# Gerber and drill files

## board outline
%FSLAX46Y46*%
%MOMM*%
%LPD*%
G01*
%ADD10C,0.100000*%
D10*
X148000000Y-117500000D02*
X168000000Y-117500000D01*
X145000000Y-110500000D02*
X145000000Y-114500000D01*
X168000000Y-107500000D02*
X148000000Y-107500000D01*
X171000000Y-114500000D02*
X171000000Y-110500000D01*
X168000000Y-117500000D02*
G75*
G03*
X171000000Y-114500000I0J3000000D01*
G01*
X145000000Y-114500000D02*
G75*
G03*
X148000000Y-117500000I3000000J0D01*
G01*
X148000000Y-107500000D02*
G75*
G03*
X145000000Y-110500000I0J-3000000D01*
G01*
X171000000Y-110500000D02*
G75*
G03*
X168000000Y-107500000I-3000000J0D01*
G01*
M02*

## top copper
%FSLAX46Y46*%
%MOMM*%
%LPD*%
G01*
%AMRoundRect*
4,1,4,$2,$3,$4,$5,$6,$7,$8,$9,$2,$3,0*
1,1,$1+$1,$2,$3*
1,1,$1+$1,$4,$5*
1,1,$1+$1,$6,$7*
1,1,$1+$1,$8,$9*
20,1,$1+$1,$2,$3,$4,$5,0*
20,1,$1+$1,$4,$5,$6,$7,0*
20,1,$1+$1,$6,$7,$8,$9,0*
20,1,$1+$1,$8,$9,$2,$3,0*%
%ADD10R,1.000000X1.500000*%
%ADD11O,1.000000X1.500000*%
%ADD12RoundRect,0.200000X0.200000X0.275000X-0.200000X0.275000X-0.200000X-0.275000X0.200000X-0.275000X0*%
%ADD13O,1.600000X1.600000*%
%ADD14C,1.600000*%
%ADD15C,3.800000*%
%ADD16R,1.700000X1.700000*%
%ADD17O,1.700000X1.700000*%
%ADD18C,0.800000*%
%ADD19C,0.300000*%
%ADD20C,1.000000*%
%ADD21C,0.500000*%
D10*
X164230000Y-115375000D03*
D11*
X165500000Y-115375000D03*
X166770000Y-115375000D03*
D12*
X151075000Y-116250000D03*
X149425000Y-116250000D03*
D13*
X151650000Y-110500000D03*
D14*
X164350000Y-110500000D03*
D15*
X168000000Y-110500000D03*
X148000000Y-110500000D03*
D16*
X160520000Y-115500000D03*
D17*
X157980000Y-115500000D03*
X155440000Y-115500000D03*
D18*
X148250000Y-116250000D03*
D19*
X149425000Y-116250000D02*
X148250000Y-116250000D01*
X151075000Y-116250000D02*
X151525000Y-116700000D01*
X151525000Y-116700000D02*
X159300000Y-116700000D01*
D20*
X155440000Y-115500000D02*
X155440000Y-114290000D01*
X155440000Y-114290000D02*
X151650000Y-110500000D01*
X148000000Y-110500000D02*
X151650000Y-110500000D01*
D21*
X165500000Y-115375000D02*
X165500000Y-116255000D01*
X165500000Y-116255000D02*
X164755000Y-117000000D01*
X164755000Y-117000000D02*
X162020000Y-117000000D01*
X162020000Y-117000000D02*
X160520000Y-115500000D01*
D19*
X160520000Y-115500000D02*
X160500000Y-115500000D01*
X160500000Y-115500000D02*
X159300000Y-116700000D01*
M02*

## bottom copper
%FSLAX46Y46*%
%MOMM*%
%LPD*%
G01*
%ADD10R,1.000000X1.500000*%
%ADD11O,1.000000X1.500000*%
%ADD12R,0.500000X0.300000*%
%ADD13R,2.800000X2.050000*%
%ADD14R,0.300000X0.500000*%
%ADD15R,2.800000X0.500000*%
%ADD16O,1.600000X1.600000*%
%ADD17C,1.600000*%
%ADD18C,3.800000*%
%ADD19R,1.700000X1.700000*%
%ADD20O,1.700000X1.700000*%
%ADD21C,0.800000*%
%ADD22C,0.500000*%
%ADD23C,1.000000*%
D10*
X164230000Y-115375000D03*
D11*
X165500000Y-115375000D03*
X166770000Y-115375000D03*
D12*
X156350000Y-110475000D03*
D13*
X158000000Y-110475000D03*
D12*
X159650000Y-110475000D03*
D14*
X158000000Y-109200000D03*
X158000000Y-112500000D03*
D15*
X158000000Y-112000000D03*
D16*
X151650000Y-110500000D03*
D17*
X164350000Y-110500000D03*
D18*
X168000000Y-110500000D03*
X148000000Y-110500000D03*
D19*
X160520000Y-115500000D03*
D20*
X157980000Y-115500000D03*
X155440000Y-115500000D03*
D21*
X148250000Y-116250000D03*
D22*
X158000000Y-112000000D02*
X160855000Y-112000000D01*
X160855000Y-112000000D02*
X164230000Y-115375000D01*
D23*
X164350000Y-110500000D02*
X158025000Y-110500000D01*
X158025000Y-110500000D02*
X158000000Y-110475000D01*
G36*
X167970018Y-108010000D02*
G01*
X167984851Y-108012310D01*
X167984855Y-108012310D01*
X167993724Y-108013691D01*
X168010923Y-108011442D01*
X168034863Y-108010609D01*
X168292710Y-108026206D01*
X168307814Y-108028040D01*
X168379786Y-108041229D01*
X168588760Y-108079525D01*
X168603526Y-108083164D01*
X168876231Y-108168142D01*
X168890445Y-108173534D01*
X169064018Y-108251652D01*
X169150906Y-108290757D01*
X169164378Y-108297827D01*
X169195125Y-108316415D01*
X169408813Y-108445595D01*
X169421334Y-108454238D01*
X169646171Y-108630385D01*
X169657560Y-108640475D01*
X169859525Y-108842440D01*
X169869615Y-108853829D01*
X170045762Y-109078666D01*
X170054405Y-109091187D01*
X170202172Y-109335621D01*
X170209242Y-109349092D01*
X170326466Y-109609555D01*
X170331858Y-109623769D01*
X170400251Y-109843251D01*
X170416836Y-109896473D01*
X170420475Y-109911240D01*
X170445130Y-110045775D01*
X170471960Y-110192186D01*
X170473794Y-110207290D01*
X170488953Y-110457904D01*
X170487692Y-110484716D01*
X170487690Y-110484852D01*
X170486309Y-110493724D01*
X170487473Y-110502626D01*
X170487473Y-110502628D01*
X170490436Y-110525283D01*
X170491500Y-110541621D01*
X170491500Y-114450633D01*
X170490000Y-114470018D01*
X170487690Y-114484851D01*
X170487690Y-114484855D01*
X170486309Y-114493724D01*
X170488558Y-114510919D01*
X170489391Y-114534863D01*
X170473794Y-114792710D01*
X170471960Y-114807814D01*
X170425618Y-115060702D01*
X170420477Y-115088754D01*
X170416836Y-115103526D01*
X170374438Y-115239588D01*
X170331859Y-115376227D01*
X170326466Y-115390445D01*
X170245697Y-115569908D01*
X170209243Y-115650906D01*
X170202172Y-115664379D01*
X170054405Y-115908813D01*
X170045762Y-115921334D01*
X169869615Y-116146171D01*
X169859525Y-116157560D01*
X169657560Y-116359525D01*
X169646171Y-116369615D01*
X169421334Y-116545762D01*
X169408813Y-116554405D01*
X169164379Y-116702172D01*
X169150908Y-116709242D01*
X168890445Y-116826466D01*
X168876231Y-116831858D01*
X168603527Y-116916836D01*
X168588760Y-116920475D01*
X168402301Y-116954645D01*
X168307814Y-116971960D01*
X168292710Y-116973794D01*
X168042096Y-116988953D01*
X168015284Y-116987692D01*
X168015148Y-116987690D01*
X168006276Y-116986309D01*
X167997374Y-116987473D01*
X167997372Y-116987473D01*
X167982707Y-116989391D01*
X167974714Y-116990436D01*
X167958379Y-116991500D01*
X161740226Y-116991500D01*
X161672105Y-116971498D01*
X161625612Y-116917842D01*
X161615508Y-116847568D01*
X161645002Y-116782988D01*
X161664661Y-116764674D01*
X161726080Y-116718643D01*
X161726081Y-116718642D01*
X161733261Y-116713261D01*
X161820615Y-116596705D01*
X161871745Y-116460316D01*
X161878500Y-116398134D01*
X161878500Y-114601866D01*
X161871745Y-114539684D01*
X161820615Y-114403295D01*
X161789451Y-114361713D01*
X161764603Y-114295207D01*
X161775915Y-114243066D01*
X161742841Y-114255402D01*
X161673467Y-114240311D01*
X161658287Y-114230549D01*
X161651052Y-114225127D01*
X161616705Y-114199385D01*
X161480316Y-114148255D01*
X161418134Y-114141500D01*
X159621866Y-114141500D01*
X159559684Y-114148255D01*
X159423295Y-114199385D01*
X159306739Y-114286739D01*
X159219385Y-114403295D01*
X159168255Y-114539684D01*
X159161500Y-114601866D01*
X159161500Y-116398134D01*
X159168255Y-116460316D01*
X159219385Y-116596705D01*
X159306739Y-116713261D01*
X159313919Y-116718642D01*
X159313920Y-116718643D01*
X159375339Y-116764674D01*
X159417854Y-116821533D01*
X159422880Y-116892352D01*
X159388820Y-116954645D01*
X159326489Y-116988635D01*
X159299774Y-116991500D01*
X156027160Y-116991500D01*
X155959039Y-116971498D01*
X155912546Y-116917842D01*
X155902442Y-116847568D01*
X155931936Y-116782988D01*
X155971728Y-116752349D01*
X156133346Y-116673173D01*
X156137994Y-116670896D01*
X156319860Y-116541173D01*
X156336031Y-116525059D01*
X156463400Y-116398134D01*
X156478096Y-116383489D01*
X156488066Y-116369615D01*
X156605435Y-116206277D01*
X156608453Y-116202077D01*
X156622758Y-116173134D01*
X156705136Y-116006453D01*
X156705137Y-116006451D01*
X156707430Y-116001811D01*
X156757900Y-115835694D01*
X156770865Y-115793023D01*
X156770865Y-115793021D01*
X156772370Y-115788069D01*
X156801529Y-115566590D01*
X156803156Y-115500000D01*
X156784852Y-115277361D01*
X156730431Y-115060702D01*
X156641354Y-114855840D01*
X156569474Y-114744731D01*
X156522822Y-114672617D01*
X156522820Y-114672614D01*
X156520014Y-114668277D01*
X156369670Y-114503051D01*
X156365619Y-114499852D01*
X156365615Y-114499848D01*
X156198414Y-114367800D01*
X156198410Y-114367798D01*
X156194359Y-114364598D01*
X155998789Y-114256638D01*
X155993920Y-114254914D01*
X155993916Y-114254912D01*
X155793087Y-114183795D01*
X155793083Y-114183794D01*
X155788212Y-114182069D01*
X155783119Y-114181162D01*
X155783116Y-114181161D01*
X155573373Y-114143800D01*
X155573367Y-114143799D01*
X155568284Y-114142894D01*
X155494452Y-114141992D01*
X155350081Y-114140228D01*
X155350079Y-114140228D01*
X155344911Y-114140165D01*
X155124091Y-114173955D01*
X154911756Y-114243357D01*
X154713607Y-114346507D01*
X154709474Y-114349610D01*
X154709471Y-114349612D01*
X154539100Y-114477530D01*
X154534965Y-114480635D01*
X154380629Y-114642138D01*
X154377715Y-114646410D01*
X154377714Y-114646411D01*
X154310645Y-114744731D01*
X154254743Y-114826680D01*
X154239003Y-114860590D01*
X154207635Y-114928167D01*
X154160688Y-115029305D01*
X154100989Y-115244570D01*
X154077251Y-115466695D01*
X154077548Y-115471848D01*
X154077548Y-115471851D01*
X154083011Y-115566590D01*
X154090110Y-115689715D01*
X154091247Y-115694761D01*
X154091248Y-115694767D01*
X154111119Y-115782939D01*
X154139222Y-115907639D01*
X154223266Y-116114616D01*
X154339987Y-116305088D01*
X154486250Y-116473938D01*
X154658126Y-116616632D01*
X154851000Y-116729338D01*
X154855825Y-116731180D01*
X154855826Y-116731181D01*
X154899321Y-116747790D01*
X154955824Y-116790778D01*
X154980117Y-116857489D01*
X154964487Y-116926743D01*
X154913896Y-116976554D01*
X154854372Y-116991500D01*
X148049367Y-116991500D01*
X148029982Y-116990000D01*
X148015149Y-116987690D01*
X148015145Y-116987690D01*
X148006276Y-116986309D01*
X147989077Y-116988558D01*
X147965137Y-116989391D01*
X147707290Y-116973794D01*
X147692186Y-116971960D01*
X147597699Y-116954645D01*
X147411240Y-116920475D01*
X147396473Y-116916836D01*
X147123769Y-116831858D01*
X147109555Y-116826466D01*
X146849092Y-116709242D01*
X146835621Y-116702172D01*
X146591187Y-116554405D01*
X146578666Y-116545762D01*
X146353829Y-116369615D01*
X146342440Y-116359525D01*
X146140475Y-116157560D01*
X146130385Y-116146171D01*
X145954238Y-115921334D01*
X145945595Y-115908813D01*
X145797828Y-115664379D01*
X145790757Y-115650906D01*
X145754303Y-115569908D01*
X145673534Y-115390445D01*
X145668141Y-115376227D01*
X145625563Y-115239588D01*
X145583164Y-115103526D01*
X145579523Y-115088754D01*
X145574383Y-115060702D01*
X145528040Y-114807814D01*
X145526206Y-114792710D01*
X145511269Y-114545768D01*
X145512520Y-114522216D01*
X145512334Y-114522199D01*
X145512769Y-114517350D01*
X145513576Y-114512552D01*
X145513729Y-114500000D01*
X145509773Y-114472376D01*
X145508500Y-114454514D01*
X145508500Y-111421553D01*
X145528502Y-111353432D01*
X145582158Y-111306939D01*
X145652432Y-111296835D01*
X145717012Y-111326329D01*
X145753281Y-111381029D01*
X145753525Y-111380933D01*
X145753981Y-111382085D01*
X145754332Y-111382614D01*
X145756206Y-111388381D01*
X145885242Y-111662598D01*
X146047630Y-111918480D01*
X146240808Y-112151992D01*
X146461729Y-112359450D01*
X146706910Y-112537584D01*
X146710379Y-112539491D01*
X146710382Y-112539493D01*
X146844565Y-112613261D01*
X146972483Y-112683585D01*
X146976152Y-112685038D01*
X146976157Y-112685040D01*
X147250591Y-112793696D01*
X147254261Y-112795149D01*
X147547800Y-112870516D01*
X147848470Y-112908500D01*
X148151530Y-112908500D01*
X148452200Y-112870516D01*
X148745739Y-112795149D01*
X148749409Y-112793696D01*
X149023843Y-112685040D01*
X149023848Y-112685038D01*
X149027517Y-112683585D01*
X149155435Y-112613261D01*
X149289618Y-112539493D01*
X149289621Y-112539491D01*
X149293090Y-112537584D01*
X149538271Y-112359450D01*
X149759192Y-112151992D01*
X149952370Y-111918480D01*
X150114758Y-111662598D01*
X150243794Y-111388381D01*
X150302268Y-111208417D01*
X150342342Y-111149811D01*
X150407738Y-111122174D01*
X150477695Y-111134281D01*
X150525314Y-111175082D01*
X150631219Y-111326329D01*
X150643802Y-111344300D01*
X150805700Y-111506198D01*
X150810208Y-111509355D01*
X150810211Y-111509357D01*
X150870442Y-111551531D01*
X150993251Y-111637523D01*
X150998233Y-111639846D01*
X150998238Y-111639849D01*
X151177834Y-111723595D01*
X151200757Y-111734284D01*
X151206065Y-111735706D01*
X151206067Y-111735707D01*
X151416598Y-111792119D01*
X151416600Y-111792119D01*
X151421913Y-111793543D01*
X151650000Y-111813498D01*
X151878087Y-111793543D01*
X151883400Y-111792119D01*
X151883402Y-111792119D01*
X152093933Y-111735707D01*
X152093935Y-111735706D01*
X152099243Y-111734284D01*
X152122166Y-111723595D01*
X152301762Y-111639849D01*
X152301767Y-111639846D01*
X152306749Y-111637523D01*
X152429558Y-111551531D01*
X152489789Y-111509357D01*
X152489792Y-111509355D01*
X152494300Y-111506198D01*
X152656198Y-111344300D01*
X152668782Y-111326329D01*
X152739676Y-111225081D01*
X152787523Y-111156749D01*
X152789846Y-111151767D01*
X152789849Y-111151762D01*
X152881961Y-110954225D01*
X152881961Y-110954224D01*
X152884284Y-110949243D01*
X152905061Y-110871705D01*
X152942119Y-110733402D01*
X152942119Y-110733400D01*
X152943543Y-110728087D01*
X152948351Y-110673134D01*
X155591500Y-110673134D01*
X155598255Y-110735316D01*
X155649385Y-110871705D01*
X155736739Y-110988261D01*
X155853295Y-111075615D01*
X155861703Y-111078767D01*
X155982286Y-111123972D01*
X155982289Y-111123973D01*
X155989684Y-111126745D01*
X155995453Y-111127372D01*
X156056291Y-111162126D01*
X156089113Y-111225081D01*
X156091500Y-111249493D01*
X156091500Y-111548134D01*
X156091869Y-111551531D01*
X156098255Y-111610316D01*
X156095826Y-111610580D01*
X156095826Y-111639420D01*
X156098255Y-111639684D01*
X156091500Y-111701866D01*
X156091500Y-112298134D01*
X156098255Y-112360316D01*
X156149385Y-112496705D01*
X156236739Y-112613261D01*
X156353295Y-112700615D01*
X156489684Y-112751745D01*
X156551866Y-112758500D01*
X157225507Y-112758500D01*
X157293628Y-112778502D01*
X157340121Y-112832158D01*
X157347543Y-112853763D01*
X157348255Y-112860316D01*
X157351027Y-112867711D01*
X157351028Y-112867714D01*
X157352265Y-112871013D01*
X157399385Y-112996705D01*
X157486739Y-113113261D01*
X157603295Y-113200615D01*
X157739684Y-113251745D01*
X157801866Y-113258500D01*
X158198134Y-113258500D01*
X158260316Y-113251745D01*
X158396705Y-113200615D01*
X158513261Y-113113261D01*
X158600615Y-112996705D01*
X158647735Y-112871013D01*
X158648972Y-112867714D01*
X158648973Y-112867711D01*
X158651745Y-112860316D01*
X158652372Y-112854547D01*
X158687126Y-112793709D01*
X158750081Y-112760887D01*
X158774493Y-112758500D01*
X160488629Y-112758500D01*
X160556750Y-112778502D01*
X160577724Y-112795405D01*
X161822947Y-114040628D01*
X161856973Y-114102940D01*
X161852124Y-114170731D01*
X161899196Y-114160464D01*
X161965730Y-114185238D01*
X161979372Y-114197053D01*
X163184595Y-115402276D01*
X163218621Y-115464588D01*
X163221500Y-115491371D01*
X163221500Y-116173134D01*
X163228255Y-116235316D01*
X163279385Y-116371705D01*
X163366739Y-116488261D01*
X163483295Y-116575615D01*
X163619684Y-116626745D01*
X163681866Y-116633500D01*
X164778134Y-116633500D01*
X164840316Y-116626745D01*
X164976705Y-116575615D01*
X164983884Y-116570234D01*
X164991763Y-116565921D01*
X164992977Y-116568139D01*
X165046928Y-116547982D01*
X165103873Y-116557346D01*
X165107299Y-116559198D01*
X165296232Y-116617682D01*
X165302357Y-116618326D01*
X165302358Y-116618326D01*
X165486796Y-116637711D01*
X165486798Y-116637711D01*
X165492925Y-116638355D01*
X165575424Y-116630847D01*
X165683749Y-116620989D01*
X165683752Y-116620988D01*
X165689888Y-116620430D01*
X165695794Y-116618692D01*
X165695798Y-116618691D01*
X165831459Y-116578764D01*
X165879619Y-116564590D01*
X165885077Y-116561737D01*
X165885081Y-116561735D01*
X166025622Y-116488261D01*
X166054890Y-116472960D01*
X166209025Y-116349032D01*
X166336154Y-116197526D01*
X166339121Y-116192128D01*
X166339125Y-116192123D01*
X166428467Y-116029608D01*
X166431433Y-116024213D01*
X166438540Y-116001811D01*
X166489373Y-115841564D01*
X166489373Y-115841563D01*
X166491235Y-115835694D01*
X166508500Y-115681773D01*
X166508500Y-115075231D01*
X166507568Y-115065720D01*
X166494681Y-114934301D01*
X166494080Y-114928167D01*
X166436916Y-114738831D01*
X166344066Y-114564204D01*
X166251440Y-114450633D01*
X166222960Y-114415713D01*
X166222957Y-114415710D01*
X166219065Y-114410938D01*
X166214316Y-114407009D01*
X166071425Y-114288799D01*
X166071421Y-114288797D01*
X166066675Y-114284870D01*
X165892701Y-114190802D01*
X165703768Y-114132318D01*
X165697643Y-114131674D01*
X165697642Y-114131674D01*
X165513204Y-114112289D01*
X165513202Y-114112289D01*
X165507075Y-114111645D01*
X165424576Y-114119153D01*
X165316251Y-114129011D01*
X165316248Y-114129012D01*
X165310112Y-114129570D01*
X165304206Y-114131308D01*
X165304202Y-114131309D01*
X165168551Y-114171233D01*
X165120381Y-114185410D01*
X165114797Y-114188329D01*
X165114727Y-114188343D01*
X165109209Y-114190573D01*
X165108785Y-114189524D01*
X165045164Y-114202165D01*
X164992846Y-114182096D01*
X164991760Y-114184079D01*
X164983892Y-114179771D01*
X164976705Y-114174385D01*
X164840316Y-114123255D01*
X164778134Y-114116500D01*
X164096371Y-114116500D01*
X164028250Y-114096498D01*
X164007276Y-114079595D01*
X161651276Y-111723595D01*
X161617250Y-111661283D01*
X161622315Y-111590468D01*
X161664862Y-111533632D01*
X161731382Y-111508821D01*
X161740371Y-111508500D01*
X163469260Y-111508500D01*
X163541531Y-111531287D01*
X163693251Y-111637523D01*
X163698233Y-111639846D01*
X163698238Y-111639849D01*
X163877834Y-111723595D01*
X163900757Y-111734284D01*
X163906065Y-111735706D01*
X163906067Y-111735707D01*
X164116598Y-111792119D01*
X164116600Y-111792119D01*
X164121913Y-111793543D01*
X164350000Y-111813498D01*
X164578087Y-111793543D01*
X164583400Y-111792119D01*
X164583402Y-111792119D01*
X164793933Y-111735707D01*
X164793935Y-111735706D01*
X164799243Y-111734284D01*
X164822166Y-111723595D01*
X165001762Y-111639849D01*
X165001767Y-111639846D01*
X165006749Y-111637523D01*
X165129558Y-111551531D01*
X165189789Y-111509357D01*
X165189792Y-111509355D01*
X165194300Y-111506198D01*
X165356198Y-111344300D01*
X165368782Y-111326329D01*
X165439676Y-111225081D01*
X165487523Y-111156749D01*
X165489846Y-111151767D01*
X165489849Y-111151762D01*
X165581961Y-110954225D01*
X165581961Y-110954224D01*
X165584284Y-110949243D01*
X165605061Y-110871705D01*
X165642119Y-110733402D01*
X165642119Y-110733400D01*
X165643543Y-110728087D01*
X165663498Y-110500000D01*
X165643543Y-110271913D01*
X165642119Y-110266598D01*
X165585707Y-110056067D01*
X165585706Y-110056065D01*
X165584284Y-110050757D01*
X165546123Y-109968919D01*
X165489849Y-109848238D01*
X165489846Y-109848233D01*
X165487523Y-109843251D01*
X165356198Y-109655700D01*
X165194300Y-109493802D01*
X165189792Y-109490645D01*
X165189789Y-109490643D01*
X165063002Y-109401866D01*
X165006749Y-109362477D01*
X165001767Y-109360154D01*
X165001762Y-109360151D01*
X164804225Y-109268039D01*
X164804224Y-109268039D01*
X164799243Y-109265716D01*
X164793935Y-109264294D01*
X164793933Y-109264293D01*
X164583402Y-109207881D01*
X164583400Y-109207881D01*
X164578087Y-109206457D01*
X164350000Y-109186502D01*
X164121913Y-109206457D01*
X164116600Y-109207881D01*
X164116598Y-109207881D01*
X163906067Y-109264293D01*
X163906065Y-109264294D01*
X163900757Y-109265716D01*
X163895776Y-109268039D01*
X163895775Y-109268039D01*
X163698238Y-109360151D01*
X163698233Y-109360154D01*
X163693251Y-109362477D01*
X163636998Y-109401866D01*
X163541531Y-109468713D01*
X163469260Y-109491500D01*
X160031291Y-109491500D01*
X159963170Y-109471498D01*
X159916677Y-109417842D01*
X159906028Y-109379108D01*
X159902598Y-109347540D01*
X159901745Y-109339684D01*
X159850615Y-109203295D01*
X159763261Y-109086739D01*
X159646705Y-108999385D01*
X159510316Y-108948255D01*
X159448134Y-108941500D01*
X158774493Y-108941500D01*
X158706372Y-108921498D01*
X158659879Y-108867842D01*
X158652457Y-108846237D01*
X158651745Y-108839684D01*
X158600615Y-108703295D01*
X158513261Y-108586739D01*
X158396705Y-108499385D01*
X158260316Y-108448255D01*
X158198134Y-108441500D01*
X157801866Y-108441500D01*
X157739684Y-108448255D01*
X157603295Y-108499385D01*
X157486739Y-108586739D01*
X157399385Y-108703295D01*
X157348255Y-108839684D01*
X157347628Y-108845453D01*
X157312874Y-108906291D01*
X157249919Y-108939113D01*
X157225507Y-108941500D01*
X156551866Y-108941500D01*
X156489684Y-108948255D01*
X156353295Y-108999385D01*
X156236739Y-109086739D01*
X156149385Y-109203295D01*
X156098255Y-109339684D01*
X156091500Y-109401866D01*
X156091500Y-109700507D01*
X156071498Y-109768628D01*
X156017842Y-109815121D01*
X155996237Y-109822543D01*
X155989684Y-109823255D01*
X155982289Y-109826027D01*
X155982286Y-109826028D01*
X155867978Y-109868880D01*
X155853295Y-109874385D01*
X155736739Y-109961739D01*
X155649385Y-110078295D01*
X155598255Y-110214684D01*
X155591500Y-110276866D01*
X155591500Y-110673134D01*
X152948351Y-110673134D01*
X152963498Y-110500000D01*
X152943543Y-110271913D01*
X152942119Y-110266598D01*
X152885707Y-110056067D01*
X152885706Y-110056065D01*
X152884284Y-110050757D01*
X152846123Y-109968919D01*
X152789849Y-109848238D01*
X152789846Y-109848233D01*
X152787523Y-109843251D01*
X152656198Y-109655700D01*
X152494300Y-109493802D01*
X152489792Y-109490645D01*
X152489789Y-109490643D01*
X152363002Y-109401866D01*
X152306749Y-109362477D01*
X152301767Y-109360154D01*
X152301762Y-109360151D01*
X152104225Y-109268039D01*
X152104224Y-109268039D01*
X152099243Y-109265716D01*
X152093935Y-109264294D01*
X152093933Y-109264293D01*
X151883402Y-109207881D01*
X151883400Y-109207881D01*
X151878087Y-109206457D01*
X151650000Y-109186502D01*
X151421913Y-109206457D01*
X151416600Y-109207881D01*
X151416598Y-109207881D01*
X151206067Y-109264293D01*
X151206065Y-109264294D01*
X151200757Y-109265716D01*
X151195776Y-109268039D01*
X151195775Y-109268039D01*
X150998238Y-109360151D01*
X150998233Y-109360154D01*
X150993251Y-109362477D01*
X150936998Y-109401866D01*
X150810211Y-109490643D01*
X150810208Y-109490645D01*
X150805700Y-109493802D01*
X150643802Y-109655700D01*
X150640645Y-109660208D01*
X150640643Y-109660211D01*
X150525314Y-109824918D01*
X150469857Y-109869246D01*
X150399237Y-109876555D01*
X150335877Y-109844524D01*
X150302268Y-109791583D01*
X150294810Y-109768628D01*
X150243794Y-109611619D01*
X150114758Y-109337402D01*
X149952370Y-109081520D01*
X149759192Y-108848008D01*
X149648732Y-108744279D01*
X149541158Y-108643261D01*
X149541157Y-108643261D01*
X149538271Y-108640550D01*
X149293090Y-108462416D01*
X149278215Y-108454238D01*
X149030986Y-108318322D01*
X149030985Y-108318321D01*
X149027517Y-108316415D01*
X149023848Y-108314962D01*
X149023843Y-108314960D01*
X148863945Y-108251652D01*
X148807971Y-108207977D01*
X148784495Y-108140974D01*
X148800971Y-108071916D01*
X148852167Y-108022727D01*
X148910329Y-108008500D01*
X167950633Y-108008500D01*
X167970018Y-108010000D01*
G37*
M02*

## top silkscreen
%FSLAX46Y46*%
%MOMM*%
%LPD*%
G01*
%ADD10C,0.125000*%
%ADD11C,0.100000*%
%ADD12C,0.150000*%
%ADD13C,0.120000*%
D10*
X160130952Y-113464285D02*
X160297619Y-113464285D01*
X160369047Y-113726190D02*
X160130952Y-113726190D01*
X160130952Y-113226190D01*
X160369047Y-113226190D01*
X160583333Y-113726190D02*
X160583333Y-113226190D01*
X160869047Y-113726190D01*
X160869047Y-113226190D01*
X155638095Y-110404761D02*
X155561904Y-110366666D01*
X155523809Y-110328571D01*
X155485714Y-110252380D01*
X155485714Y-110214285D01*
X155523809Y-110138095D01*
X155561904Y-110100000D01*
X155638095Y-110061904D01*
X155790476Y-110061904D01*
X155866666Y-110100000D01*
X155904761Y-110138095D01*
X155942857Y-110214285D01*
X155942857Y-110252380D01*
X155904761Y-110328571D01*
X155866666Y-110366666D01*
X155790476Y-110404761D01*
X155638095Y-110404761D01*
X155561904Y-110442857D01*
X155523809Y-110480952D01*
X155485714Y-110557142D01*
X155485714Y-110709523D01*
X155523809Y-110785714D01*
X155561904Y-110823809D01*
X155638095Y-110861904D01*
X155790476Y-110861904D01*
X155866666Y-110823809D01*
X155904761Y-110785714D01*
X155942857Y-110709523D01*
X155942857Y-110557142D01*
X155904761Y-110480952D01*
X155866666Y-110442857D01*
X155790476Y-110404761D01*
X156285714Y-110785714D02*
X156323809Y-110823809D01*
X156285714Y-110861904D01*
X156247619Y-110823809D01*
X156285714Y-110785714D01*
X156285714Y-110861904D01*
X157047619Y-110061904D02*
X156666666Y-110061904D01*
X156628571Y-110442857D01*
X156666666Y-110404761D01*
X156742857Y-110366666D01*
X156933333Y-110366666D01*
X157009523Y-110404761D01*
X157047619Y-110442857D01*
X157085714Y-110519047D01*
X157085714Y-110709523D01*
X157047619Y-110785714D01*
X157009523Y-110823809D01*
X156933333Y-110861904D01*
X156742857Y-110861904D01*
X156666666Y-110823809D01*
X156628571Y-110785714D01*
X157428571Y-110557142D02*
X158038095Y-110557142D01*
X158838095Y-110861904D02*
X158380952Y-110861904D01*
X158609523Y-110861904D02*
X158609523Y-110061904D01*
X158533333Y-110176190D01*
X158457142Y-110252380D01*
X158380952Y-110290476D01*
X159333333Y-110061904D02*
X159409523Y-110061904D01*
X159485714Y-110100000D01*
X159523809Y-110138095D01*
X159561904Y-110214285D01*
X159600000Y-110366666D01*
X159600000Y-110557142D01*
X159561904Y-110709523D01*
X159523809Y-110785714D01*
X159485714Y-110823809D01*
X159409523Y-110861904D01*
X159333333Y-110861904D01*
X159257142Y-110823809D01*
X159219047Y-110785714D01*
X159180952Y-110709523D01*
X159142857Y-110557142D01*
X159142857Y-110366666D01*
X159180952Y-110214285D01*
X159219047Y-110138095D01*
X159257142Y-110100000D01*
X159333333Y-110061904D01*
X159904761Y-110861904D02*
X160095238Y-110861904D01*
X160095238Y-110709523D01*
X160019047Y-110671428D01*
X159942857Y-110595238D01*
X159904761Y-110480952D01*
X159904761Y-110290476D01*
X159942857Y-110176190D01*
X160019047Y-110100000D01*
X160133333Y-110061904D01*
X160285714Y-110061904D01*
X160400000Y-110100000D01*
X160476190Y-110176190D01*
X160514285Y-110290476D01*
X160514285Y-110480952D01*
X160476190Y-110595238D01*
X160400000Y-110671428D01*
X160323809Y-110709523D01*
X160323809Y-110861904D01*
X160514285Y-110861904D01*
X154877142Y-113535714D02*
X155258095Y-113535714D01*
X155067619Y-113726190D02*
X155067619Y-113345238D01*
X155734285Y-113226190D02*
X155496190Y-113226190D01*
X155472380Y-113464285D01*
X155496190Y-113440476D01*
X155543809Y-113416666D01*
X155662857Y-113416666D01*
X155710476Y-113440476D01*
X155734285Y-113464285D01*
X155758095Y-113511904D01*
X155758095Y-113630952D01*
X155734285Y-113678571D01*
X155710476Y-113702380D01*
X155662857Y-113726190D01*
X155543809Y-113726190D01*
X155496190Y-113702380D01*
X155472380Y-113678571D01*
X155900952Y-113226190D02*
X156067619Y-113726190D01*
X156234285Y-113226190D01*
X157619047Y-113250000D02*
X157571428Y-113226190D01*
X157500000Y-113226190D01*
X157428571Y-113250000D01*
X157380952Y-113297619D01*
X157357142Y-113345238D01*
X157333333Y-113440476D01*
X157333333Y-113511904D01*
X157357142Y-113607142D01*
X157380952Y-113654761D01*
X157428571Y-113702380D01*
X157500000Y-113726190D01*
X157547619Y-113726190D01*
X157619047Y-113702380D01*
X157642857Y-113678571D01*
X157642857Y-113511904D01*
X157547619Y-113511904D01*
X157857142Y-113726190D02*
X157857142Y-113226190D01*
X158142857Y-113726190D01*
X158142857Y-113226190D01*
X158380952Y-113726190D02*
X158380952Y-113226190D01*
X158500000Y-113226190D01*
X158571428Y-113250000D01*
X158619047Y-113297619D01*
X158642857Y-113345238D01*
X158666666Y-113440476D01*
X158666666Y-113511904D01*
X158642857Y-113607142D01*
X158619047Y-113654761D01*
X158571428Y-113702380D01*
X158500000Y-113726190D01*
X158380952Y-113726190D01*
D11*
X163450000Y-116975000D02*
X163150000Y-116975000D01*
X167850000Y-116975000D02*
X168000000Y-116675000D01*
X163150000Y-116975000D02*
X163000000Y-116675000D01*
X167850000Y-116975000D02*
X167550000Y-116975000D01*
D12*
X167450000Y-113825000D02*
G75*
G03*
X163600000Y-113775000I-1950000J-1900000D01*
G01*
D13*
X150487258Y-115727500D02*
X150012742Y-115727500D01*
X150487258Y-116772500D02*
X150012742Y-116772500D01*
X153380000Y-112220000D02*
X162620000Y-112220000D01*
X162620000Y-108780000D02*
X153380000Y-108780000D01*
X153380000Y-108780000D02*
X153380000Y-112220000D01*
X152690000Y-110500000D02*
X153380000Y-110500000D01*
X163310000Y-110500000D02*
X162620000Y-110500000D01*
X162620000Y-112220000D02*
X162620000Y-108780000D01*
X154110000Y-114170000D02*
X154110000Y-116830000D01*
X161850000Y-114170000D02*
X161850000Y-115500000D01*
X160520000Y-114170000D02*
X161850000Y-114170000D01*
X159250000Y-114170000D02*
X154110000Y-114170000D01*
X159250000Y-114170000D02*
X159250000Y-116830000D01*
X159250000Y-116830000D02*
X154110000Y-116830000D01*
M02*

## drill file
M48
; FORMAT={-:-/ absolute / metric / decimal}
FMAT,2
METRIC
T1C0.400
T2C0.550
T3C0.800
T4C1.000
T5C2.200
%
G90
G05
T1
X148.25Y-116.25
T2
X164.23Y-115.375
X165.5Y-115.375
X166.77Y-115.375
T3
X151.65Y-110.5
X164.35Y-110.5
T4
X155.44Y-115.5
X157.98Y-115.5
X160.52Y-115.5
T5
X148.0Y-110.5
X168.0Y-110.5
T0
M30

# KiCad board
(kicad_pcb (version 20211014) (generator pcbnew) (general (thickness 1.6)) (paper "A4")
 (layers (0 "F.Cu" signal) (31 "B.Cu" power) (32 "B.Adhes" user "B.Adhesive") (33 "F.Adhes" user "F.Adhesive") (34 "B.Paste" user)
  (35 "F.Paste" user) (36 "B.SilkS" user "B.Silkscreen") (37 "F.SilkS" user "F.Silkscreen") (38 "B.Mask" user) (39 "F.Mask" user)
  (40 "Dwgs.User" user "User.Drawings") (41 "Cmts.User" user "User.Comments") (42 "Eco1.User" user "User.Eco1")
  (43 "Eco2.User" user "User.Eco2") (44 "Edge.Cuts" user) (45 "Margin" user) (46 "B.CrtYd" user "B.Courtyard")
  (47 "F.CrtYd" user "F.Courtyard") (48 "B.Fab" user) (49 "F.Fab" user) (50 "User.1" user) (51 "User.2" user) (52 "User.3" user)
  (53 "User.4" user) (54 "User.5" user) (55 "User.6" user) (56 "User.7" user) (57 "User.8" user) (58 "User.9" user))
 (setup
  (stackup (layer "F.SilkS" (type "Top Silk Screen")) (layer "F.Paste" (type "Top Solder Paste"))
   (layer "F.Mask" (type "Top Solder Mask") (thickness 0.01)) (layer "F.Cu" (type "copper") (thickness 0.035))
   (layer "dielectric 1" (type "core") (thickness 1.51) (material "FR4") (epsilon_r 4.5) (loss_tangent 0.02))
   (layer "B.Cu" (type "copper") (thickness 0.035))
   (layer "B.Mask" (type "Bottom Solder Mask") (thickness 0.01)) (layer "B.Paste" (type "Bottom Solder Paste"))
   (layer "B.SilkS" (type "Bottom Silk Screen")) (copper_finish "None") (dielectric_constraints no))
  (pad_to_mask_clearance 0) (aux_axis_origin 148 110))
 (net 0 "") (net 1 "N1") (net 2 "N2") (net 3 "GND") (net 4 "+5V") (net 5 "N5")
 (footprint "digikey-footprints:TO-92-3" (layer "F.Cu") (at 164.23 115.375)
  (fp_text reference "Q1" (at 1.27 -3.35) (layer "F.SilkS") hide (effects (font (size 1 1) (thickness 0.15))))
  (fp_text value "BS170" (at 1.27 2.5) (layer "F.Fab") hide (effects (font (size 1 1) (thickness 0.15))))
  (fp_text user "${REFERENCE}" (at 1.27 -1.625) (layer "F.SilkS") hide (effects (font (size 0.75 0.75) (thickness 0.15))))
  (fp_line (start -0.78 1.6) (end -1.08 1.6) (layer "F.SilkS") (width 0.1))
  (fp_line (start 3.62 1.6) (end 3.77 1.3) (layer "F.SilkS") (width 0.1))
  (fp_line (start -1.08 1.6) (end -1.23 1.3) (layer "F.SilkS") (width 0.1))
  (fp_line (start 3.62 1.6) (end 3.32 1.6) (layer "F.SilkS") (width 0.1))
  (fp_arc (start -0.63 -1.6) (mid 1.305355 -2.372361) (end 3.22 -1.55) (layer "F.SilkS") (width 0.15))
  (pad "1" thru_hole rect locked (at 0 0 180) (size 1 1.5) (drill 0.55) (layers *.Cu *.Mask) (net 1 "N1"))
  (pad "2" thru_hole oval locked (at 1.27 0 180) (size 1 1.5) (drill 0.55) (layers *.Cu *.Mask) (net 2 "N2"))
  (pad "3" thru_hole oval locked (at 2.54 0 180) (size 1 1.5) (drill 0.55) (layers *.Cu *.Mask) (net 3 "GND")))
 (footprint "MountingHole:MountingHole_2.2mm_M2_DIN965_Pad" (layer "F.Cu") (at 168 110.5)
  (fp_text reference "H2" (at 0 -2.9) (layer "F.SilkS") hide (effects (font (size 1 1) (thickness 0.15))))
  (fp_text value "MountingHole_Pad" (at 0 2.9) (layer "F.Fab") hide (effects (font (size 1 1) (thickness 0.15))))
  (pad "1" thru_hole circle (at 0 0) (size 3.8 3.8) (drill 2.2) (layers *.Cu *.Mask) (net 3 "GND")))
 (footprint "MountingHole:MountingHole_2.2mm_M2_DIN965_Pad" (layer "F.Cu") (at 148 110.5)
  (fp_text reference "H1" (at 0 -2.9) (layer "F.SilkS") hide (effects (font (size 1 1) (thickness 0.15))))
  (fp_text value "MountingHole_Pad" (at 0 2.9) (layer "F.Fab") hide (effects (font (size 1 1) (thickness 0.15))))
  (pad "1" thru_hole circle (at 0 0) (size 3.8 3.8) (drill 2.2) (layers *.Cu *.Mask) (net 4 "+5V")))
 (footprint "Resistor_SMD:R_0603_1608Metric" (layer "F.Cu") (at 150.25 116.25 180)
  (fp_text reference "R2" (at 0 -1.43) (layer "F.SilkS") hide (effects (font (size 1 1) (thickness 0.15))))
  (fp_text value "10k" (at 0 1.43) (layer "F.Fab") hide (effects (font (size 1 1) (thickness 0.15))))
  (fp_line (start -0.237258 0.5225) (end 0.237258 0.5225) (layer "F.SilkS") (width 0.12))
  (fp_line (start -0.237258 -0.5225) (end 0.237258 -0.5225) (layer "F.SilkS") (width 0.12))
  (pad "1" smd roundrect (at -0.825 0 180) (size 0.8 0.95) (layers "F.Cu" "F.Paste" "F.Mask") (roundrect_rratio 0.25) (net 2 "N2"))
  (pad "2" smd roundrect (at 0.825 0 180) (size 0.8 0.95) (layers "F.Cu" "F.Paste" "F.Mask") (roundrect_rratio 0.25) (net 3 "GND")))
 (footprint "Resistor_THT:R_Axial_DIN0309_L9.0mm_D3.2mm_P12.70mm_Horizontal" (layer "F.Cu") (at 164.35 110.5 180)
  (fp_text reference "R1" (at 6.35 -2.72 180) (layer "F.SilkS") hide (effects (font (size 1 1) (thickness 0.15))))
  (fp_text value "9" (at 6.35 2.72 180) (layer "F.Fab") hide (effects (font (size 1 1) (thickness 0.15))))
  (fp_line (start 10.97 -1.72) (end 1.73 -1.72) (layer "F.SilkS") (width 0.12))
  (fp_line (start 1.04 0) (end 1.73 0) (layer "F.SilkS") (width 0.12))
  (fp_line (start 1.73 1.72) (end 10.97 1.72) (layer "F.SilkS") (width 0.12))
  (fp_line (start 1.73 -1.72) (end 1.73 1.72) (layer "F.SilkS") (width 0.12))
  (fp_line (start 11.66 0) (end 10.97 0) (layer "F.SilkS") (width 0.12))
  (fp_line (start 10.97 1.72) (end 10.97 -1.72) (layer "F.SilkS") (width 0.12))
  (pad "1" thru_hole circle (at 0 0 180) (size 1.6 1.6) (drill 0.8) (layers *.Cu *.Mask) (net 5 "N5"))
  (pad "2" thru_hole oval (at 12.7 0 180) (size 1.6 1.6) (drill 0.8) (layers *.Cu *.Mask) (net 4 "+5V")))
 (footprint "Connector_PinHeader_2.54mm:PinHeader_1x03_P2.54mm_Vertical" (layer "F.Cu") (at 160.52 115.5 -90)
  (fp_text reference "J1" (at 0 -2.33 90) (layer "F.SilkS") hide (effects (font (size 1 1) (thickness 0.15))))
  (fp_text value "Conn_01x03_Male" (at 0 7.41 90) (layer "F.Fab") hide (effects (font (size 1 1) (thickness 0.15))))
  (fp_line (start -1.33 6.41) (end 1.33 6.41) (layer "F.SilkS") (width 0.12))
  (fp_line (start -1.33 -1.33) (end 0 -1.33) (layer "F.SilkS") (width 0.12))
  (fp_line (start -1.33 0) (end -1.33 -1.33) (layer "F.SilkS") (width 0.12))
  (fp_line (start -1.33 1.27) (end -1.33 6.41) (layer "F.SilkS") (width 0.12))
  (fp_line (start -1.33 1.27) (end 1.33 1.27) (layer "F.SilkS") (width 0.12))
  (fp_line (start 1.33 1.27) (end 1.33 6.41) (layer "F.SilkS") (width 0.12))
  (pad "1" thru_hole rect (at 0 0 270) (size 1.7 1.7) (drill 1) (layers *.Cu *.Mask) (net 2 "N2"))
  (pad "2" thru_hole oval (at 0 2.54 270) (size 1.7 1.7) (drill 1) (layers *.Cu *.Mask) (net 3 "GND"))
  (pad "3" thru_hole oval (at 0 5.08 270) (size 1.7 1.7) (drill 1) (layers *.Cu *.Mask) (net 4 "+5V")))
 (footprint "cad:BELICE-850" (layer "B.Cu") (at 158 110.475 -90)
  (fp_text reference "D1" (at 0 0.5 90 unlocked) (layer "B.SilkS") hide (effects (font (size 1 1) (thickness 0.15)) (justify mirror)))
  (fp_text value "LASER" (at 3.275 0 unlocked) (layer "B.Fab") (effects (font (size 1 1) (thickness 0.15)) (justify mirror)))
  (pad "1" smd rect (at 1.525 0 270) (size 0.5 2.8) (layers "B.Cu" "B.Paste" "B.Mask") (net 1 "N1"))
  (pad "1" smd rect (at 2.025 0 90) (size 0.5 0.3) (layers "B.Cu" "B.Paste" "B.Mask") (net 1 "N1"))
  (pad "2" smd rect (at -1.275 0 270) (size 0.5 0.3) (layers "B.Cu" "B.Paste" "B.Mask") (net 5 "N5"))
  (pad "2" smd rect (at 0 -1.65 180) (size 0.5 0.3) (layers "B.Cu" "B.Paste" "B.Mask") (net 5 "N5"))
  (pad "2" smd rect (at 0 0 270) (size 2.05 2.8) (layers "B.Cu" "B.Paste" "B.Mask") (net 5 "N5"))
  (pad "2" smd rect (at 0 1.65 180) (size 0.5 0.3) (layers "B.Cu" "B.Paste" "B.Mask") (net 5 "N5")))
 (gr_line (start 148 117.5) (end 168 117.5) (layer "Edge.Cuts") (width 0.1))
 (gr_arc (start 145 110.5) (mid 145.87868 108.37868) (end 148 107.5) (layer "Edge.Cuts") (width 0.1))
 (gr_arc (start 148 117.5) (mid 145.87868 116.62132) (end 145 114.5) (layer "Edge.Cuts") (width 0.1))
 (gr_arc (start 171 114.5) (mid 170.12132 116.62132) (end 168 117.5) (layer "Edge.Cuts") (width 0.1))
 (gr_line (start 145 110.5) (end 145 114.5) (layer "Edge.Cuts") (width 0.1))
 (gr_line (start 171 114.5) (end 171 110.5) (layer "Edge.Cuts") (width 0.1))
 (gr_arc (start 168 107.5) (mid 170.12132 108.37868) (end 171 110.5) (layer "Edge.Cuts") (width 0.1))
 (gr_line (start 168 107.5) (end 148 107.5) (layer "Edge.Cuts") (width 0.1))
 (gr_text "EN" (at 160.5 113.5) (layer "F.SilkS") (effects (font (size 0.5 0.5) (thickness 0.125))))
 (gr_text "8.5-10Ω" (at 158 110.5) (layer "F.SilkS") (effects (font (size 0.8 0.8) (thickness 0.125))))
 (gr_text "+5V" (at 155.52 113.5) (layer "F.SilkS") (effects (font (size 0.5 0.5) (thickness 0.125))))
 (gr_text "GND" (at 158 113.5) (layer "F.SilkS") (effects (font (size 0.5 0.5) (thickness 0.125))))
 (segment (start 160.855 112) (end 164.23 115.375) (width 0.5) (layer "B.Cu") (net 1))
 (segment (start 158 112) (end 160.855 112) (width 0.5) (layer "B.Cu") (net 1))
 (segment (start 158.025 110.5) (end 158 110.475) (width 1) (layer "B.Cu") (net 5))
 (segment (start 164.35 110.5) (end 158.025 110.5) (width 1) (layer "B.Cu") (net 5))
 (segment (start 149.425 116.25) (end 148.25 116.25) (width 0.3) (layer "F.Cu") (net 3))
 (via (at 148.25 116.25) (size 0.8) (drill 0.4) (layers "F.Cu" "B.Cu") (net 3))
 (segment (start 155.44 115.5) (end 155.44 114.29) (width 1) (layer "F.Cu") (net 4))
 (segment (start 148 110.5) (end 151.65 110.5) (width 1) (layer "F.Cu") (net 4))
 (segment (start 155.44 114.29) (end 151.65 110.5) (width 1) (layer "F.Cu") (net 4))
 (segment (start 160.5 115.5) (end 159.3 116.7) (width 0.3) (layer "F.Cu") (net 2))
 (segment (start 151.075 116.25) (end 151.525 116.7) (width 0.3) (layer "F.Cu") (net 2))
 (segment (start 165.5 115.375) (end 165.5 116.255) (width 0.5) (layer "F.Cu") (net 2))
 (segment (start 164.755 117) (end 162.02 117) (width 0.5) (layer "F.Cu") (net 2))
 (segment (start 162.02 117) (end 160.52 115.5) (width 0.5) (layer "F.Cu") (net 2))
 (segment (start 151.525 116.7) (end 159.3 116.7) (width 0.3) (layer "F.Cu") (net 2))
 (segment (start 160.52 115.5) (end 160.5 115.5) (width 0.3) (layer "F.Cu") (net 2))
 (segment (start 165.5 116.255) (end 164.755 117) (width 0.5) (layer "F.Cu") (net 2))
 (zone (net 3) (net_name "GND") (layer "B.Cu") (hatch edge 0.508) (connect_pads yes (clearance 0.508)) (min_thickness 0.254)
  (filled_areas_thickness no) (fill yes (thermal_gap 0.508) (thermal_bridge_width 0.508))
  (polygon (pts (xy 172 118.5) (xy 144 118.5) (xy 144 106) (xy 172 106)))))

